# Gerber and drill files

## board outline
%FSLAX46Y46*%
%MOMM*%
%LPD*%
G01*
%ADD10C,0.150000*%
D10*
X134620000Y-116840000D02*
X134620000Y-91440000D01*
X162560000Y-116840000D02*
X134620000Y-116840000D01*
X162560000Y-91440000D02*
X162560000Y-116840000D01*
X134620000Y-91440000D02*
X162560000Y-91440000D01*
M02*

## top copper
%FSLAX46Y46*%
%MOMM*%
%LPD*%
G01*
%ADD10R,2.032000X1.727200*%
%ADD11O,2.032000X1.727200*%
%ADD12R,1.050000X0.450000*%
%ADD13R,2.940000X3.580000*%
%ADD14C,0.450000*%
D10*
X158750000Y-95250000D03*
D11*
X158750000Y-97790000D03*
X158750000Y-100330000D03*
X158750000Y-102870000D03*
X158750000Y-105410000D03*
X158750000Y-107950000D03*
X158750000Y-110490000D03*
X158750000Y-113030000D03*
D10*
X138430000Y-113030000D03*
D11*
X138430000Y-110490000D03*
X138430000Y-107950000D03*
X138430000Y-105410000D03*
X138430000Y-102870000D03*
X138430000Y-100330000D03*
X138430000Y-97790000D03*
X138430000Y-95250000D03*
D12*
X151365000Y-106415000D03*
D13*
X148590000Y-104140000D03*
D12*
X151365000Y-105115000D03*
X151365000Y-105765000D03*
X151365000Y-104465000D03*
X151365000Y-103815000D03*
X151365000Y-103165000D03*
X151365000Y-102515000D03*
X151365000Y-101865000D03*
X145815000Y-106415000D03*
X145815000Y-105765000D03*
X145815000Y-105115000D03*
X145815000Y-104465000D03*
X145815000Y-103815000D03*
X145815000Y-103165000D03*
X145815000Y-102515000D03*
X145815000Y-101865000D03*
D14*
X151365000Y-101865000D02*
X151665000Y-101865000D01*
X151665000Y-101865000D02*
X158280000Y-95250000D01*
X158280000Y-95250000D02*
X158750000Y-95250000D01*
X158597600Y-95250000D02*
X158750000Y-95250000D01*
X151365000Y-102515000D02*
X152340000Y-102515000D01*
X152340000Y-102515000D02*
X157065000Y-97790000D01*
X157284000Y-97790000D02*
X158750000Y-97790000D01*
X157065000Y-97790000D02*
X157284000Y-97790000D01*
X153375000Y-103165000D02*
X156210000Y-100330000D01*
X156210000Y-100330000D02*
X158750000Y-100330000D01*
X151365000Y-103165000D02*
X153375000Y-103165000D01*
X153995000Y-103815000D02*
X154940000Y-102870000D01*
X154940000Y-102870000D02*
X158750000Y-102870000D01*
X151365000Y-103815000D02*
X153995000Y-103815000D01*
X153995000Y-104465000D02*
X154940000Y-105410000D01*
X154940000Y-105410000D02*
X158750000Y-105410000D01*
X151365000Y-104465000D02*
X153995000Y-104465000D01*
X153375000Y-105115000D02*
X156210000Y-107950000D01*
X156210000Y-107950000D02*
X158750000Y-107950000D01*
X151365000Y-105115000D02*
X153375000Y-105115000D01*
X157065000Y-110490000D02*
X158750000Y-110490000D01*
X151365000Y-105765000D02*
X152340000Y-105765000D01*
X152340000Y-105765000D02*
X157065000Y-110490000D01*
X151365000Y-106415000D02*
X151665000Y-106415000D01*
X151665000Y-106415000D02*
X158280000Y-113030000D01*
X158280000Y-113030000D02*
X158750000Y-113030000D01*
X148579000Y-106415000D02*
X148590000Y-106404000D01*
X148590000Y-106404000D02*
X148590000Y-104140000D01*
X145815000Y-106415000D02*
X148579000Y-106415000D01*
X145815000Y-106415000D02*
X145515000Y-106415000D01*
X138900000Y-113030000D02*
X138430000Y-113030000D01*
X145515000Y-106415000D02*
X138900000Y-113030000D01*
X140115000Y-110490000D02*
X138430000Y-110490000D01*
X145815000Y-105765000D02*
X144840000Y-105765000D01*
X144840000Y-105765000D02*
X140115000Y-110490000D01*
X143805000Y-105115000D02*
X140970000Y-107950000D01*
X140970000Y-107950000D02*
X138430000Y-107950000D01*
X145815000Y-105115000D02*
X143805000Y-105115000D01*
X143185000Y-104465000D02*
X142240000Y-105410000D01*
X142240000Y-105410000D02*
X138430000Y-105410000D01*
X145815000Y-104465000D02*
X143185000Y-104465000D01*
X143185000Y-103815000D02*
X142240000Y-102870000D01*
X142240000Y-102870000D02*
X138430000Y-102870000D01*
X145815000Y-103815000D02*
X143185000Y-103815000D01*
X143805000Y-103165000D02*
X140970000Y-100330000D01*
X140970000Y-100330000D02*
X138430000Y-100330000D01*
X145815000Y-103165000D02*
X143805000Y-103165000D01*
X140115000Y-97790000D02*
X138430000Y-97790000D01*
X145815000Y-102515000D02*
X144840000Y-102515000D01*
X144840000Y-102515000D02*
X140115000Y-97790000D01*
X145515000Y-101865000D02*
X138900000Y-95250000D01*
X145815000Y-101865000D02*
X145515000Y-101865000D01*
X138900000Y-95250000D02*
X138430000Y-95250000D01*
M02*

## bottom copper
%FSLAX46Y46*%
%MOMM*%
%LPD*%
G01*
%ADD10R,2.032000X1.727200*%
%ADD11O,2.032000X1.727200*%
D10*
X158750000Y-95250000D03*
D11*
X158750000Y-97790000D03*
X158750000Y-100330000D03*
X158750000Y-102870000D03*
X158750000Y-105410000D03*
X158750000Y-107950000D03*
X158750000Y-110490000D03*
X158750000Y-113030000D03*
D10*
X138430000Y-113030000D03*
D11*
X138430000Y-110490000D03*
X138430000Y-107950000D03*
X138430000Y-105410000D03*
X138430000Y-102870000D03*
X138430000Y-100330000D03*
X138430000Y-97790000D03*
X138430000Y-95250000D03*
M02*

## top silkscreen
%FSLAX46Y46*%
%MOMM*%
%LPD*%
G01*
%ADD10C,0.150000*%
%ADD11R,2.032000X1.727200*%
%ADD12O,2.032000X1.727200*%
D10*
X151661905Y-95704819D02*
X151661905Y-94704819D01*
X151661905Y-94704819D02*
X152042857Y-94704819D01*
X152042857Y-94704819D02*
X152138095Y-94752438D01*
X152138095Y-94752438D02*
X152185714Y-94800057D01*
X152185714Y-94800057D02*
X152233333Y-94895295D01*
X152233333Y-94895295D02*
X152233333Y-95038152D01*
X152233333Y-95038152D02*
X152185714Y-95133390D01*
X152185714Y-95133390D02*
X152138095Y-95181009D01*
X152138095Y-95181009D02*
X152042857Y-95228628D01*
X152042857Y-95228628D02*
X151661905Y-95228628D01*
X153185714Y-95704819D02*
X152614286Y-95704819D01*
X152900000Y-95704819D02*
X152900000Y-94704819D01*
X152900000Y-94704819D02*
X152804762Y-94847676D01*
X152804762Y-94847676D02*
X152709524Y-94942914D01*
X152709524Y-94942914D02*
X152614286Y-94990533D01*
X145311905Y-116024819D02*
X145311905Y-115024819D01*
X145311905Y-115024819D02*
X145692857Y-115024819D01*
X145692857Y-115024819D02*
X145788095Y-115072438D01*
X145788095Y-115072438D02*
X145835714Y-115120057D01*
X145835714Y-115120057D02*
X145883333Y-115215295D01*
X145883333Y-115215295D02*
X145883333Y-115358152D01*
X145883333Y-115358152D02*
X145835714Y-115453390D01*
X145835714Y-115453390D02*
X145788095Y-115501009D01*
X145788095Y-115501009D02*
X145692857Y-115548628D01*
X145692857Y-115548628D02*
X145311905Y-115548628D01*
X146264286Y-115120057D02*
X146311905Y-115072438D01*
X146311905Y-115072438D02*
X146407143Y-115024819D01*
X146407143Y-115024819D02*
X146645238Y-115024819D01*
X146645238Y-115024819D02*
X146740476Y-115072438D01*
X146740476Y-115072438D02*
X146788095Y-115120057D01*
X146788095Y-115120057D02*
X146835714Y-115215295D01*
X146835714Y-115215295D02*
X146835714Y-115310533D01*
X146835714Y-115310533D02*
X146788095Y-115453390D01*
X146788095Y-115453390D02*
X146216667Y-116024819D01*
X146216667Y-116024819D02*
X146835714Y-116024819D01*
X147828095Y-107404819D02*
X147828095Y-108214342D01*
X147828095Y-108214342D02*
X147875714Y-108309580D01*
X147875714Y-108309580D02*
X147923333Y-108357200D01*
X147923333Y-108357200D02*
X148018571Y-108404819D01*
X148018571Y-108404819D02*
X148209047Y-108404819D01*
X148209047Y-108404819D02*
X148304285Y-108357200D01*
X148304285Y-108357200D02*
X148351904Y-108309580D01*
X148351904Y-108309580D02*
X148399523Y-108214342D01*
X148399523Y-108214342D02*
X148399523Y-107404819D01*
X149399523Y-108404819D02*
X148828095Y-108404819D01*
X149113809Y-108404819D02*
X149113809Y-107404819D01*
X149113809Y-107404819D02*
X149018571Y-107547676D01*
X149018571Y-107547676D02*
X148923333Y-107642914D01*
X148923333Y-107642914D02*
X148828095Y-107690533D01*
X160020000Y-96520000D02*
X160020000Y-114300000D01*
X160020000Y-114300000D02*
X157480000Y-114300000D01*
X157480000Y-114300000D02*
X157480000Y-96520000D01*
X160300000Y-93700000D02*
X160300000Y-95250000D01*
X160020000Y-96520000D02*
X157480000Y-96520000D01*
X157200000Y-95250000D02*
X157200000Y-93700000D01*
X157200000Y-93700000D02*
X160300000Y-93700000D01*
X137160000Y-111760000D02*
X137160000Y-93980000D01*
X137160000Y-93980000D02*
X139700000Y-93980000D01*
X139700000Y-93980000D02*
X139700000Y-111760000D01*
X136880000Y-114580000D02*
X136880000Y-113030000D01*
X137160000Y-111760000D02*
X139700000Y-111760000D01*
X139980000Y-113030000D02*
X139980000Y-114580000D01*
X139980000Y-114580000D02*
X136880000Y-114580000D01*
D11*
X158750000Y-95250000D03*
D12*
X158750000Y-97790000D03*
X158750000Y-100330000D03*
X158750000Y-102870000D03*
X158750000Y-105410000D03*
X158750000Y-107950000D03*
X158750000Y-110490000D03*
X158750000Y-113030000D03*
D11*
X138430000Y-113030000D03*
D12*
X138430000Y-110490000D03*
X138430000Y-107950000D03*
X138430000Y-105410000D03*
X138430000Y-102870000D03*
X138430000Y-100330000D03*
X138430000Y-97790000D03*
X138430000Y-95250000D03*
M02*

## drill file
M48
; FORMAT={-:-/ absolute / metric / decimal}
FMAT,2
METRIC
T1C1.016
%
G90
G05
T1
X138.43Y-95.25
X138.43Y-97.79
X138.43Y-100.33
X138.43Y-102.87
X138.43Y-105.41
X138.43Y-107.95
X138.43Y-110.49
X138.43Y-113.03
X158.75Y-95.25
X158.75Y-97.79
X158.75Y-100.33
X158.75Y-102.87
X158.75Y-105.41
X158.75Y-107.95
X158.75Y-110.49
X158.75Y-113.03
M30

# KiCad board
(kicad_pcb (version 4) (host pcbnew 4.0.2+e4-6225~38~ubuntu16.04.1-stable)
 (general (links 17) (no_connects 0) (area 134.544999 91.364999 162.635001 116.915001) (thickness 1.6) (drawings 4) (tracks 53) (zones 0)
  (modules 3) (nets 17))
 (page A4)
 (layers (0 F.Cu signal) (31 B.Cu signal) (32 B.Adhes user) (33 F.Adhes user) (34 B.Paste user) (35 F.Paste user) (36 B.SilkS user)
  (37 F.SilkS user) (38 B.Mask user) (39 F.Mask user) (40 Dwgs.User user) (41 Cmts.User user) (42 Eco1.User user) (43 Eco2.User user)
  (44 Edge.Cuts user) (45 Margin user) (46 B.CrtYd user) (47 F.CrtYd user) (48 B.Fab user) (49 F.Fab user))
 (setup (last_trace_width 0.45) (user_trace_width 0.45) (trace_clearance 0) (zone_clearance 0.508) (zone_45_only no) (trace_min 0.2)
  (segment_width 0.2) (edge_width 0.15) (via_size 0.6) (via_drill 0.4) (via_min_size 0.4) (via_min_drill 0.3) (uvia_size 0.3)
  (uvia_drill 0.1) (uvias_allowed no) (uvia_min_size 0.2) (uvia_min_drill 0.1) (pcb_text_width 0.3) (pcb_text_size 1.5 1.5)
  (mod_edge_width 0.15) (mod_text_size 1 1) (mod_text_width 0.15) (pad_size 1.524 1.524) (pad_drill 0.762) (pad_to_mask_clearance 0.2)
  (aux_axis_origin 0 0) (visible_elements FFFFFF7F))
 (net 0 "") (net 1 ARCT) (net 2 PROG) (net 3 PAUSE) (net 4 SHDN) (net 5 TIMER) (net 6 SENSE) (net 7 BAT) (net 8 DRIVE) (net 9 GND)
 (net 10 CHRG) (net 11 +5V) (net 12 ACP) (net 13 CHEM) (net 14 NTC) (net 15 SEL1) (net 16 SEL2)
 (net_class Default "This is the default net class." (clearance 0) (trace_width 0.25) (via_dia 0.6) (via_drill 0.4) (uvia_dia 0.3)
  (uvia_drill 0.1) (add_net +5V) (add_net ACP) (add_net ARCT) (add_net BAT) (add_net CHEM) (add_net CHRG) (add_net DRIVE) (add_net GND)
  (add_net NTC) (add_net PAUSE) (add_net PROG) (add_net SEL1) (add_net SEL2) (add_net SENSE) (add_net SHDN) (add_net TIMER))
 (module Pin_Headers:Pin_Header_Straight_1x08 (layer F.Cu) (at 158.75 95.25)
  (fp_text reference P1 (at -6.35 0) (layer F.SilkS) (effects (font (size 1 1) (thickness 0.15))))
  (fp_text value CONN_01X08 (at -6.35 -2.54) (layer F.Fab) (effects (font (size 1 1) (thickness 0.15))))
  (fp_line (start 1.27 1.27) (end 1.27 19.05) (layer F.SilkS) (width 0.15))
  (fp_line (start 1.27 19.05) (end -1.27 19.05) (layer F.SilkS) (width 0.15))
  (fp_line (start -1.27 19.05) (end -1.27 1.27) (layer F.SilkS) (width 0.15))
  (fp_line (start 1.55 -1.55) (end 1.55 0) (layer F.SilkS) (width 0.15))
  (fp_line (start 1.27 1.27) (end -1.27 1.27) (layer F.SilkS) (width 0.15))
  (fp_line (start -1.55 0) (end -1.55 -1.55) (layer F.SilkS) (width 0.15))
  (fp_line (start -1.55 -1.55) (end 1.55 -1.55) (layer F.SilkS) (width 0.15))
  (pad 1 thru_hole rect (at 0 0) (size 2.032 1.7272) (drill 1.016) (layers *.Cu *.Mask F.SilkS) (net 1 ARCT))
  (pad 2 thru_hole oval (at 0 2.54) (size 2.032 1.7272) (drill 1.016) (layers *.Cu *.Mask F.SilkS) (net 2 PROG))
  (pad 3 thru_hole oval (at 0 5.08) (size 2.032 1.7272) (drill 1.016) (layers *.Cu *.Mask F.SilkS) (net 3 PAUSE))
  (pad 4 thru_hole oval (at 0 7.62) (size 2.032 1.7272) (drill 1.016) (layers *.Cu *.Mask F.SilkS) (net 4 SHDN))
  (pad 5 thru_hole oval (at 0 10.16) (size 2.032 1.7272) (drill 1.016) (layers *.Cu *.Mask F.SilkS) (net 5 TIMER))
  (pad 6 thru_hole oval (at 0 12.7) (size 2.032 1.7272) (drill 1.016) (layers *.Cu *.Mask F.SilkS) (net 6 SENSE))
  (pad 7 thru_hole oval (at 0 15.24) (size 2.032 1.7272) (drill 1.016) (layers *.Cu *.Mask F.SilkS) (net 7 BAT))
  (pad 8 thru_hole oval (at 0 17.78) (size 2.032 1.7272) (drill 1.016) (layers *.Cu *.Mask F.SilkS) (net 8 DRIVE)))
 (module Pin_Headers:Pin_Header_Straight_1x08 (layer F.Cu) (at 138.43 113.03 180)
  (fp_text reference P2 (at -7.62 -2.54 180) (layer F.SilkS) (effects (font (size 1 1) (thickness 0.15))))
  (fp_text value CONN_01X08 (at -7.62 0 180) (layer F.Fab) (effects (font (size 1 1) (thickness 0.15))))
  (fp_line (start 1.27 1.27) (end 1.27 19.05) (layer F.SilkS) (width 0.15))
  (fp_line (start 1.27 19.05) (end -1.27 19.05) (layer F.SilkS) (width 0.15))
  (fp_line (start -1.27 19.05) (end -1.27 1.27) (layer F.SilkS) (width 0.15))
  (fp_line (start 1.55 -1.55) (end 1.55 0) (layer F.SilkS) (width 0.15))
  (fp_line (start 1.27 1.27) (end -1.27 1.27) (layer F.SilkS) (width 0.15))
  (fp_line (start -1.55 0) (end -1.55 -1.55) (layer F.SilkS) (width 0.15))
  (fp_line (start -1.55 -1.55) (end 1.55 -1.55) (layer F.SilkS) (width 0.15))
  (pad 1 thru_hole rect (at 0 0 180) (size 2.032 1.7272) (drill 1.016) (layers *.Cu *.Mask F.SilkS) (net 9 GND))
  (pad 2 thru_hole oval (at 0 2.54 180) (size 2.032 1.7272) (drill 1.016) (layers *.Cu *.Mask F.SilkS) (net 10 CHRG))
  (pad 3 thru_hole oval (at 0 5.08 180) (size 2.032 1.7272) (drill 1.016) (layers *.Cu *.Mask F.SilkS) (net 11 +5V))
  (pad 4 thru_hole oval (at 0 7.62 180) (size 2.032 1.7272) (drill 1.016) (layers *.Cu *.Mask F.SilkS) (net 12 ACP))
  (pad 5 thru_hole oval (at 0 10.16 180) (size 2.032 1.7272) (drill 1.016) (layers *.Cu *.Mask F.SilkS) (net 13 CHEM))
  (pad 6 thru_hole oval (at 0 12.7 180) (size 2.032 1.7272) (drill 1.016) (layers *.Cu *.Mask F.SilkS) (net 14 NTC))
  (pad 7 thru_hole oval (at 0 15.24 180) (size 2.032 1.7272) (drill 1.016) (layers *.Cu *.Mask F.SilkS) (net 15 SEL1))
  (pad 8 thru_hole oval (at 0 17.78 180) (size 2.032 1.7272) (drill 1.016) (layers *.Cu *.Mask F.SilkS) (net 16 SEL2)))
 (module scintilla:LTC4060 (layer F.Cu) (at 148.59 104.14 90)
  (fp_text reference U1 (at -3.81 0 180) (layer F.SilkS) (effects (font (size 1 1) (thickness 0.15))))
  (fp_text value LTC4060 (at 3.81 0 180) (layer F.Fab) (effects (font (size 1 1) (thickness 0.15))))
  (pad 1 smd rect (at -2.275 2.775 90) (size 0.45 1.05) (layers F.Cu F.Paste F.Mask) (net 8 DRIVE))
  (pad 17 smd rect (at 0 0 90) (size 3.58 2.94) (layers F.Cu F.Paste F.Mask) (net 9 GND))
  (pad 3 smd rect (at -0.975 2.775 90) (size 0.45 1.05) (layers F.Cu F.Paste F.Mask) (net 6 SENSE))
  (pad 2 smd rect (at -1.625 2.775 90) (size 0.45 1.05) (layers F.Cu F.Paste F.Mask) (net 7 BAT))
  (pad 4 smd rect (at -0.325 2.775 90) (size 0.45 1.05) (layers F.Cu F.Paste F.Mask) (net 5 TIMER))
  (pad 5 smd rect (at 0.325 2.775 90) (size 0.45 1.05) (layers F.Cu F.Paste F.Mask) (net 4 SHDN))
  (pad 6 smd rect (at 0.975 2.775 90) (size 0.45 1.05) (layers F.Cu F.Paste F.Mask) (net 3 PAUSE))
  (pad 7 smd rect (at 1.625 2.775 90) (size 0.45 1.05) (layers F.Cu F.Paste F.Mask) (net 2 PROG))
  (pad 8 smd rect (at 2.275 2.775 90) (size 0.45 1.05) (layers F.Cu F.Paste F.Mask) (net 1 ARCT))
  (pad 16 smd rect (at -2.275 -2.775 90) (size 0.45 1.05) (layers F.Cu F.Paste F.Mask) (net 9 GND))
  (pad 15 smd rect (at -1.625 -2.775 90) (size 0.45 1.05) (layers F.Cu F.Paste F.Mask) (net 10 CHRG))
  (pad 14 smd rect (at -0.975 -2.775 90) (size 0.45 1.05) (layers F.Cu F.Paste F.Mask) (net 11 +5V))
  (pad 13 smd rect (at -0.325 -2.775 90) (size 0.45 1.05) (layers F.Cu F.Paste F.Mask) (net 12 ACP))
  (pad 12 smd rect (at 0.325 -2.775 90) (size 0.45 1.05) (layers F.Cu F.Paste F.Mask) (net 13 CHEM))
  (pad 11 smd rect (at 0.975 -2.775 90) (size 0.45 1.05) (layers F.Cu F.Paste F.Mask) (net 14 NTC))
  (pad 10 smd rect (at 1.625 -2.775 90) (size 0.45 1.05) (layers F.Cu F.Paste F.Mask) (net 15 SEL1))
  (pad 9 smd rect (at 2.275 -2.775 90) (size 0.45 1.05) (layers F.Cu F.Paste F.Mask) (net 16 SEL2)))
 (gr_line (start 134.62 116.84) (end 134.62 91.44) (layer Edge.Cuts) (width 0.15))
 (gr_line (start 162.56 116.84) (end 134.62 116.84) (layer Edge.Cuts) (width 0.15))
 (gr_line (start 162.56 91.44) (end 162.56 116.84) (layer Edge.Cuts) (width 0.15))
 (gr_line (start 134.62 91.44) (end 162.56 91.44) (layer Edge.Cuts) (width 0.15))
 (segment (start 151.365 101.865) (end 151.665 101.865) (width 0.45) (layer F.Cu) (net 1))
 (segment (start 151.665 101.865) (end 158.28 95.25) (width 0.45) (layer F.Cu) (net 1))
 (segment (start 158.28 95.25) (end 158.75 95.25) (width 0.45) (layer F.Cu) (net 1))
 (segment (start 158.5976 95.25) (end 158.75 95.25) (width 0.45) (layer F.Cu) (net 1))
 (segment (start 151.365 102.515) (end 152.34 102.515) (width 0.45) (layer F.Cu) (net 2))
 (segment (start 152.34 102.515) (end 157.065 97.79) (width 0.45) (layer F.Cu) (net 2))
 (segment (start 157.284 97.79) (end 158.75 97.79) (width 0.45) (layer F.Cu) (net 2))
 (segment (start 157.065 97.79) (end 157.284 97.79) (width 0.45) (layer F.Cu) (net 2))
 (segment (start 153.375 103.165) (end 156.21 100.33) (width 0.45) (layer F.Cu) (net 3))
 (segment (start 156.21 100.33) (end 158.75 100.33) (width 0.45) (layer F.Cu) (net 3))
 (segment (start 151.365 103.165) (end 153.375 103.165) (width 0.45) (layer F.Cu) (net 3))
 (segment (start 153.995 103.815) (end 154.94 102.87) (width 0.45) (layer F.Cu) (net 4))
 (segment (start 154.94 102.87) (end 158.75 102.87) (width 0.45) (layer F.Cu) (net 4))
 (segment (start 151.365 103.815) (end 153.995 103.815) (width 0.45) (layer F.Cu) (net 4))
 (segment (start 153.995 104.465) (end 154.94 105.41) (width 0.45) (layer F.Cu) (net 5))
 (segment (start 154.94 105.41) (end 158.75 105.41) (width 0.45) (layer F.Cu) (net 5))
 (segment (start 151.365 104.465) (end 153.995 104.465) (width 0.45) (layer F.Cu) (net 5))
 (segment (start 153.375 105.115) (end 156.21 107.95) (width 0.45) (layer F.Cu) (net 6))
 (segment (start 156.21 107.95) (end 158.75 107.95) (width 0.45) (layer F.Cu) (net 6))
 (segment (start 151.365 105.115) (end 153.375 105.115) (width 0.45) (layer F.Cu) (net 6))
 (segment (start 157.065 110.49) (end 158.75 110.49) (width 0.45) (layer F.Cu) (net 7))
 (segment (start 151.365 105.765) (end 152.34 105.765) (width 0.45) (layer F.Cu) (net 7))
 (segment (start 152.34 105.765) (end 157.065 110.49) (width 0.45) (layer F.Cu) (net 7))
 (segment (start 151.365 106.415) (end 151.665 106.415) (width 0.45) (layer F.Cu) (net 8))
 (segment (start 151.665 106.415) (end 158.28 113.03) (width 0.45) (layer F.Cu) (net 8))
 (segment (start 158.28 113.03) (end 158.75 113.03) (width 0.45) (layer F.Cu) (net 8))
 (segment (start 148.579 106.415) (end 148.59 106.404) (width 0.45) (layer F.Cu) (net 9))
 (segment (start 148.59 106.404) (end 148.59 104.14) (width 0.45) (layer F.Cu) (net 9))
 (segment (start 145.815 106.415) (end 148.579 106.415) (width 0.45) (layer F.Cu) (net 9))
 (segment (start 145.815 106.415) (end 145.515 106.415) (width 0.45) (layer F.Cu) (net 9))
 (segment (start 138.9 113.03) (end 138.43 113.03) (width 0.45) (layer F.Cu) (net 9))
 (segment (start 145.515 106.415) (end 138.9 113.03) (width 0.45) (layer F.Cu) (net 9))
 (segment (start 140.115 110.49) (end 138.43 110.49) (width 0.45) (layer F.Cu) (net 10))
 (segment (start 145.815 105.765) (end 144.84 105.765) (width 0.45) (layer F.Cu) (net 10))
 (segment (start 144.84 105.765) (end 140.115 110.49) (width 0.45) (layer F.Cu) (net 10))
 (segment (start 143.805 105.115) (end 140.97 107.95) (width 0.45) (layer F.Cu) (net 11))
 (segment (start 140.97 107.95) (end 138.43 107.95) (width 0.45) (layer F.Cu) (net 11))
 (segment (start 145.815 105.115) (end 143.805 105.115) (width 0.45) (layer F.Cu) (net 11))
 (segment (start 143.185 104.465) (end 142.24 105.41) (width 0.45) (layer F.Cu) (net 12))
 (segment (start 142.24 105.41) (end 138.43 105.41) (width 0.45) (layer F.Cu) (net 12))
 (segment (start 145.815 104.465) (end 143.185 104.465) (width 0.45) (layer F.Cu) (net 12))
 (segment (start 143.185 103.815) (end 142.24 102.87) (width 0.45) (layer F.Cu) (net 13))
 (segment (start 142.24 102.87) (end 138.43 102.87) (width 0.45) (layer F.Cu) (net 13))
 (segment (start 145.815 103.815) (end 143.185 103.815) (width 0.45) (layer F.Cu) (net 13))
 (segment (start 143.805 103.165) (end 140.97 100.33) (width 0.45) (layer F.Cu) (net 14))
 (segment (start 140.97 100.33) (end 138.43 100.33) (width 0.45) (layer F.Cu) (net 14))
 (segment (start 145.815 103.165) (end 143.805 103.165) (width 0.45) (layer F.Cu) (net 14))
 (segment (start 140.115 97.79) (end 138.43 97.79) (width 0.45) (layer F.Cu) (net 15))
 (segment (start 145.815 102.515) (end 144.84 102.515) (width 0.45) (layer F.Cu) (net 15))
 (segment (start 144.84 102.515) (end 140.115 97.79) (width 0.45) (layer F.Cu) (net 15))
 (segment (start 145.515 101.865) (end 138.9 95.25) (width 0.45) (layer F.Cu) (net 16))
 (segment (start 145.815 101.865) (end 145.515 101.865) (width 0.45) (layer F.Cu) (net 16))
 (segment (start 138.9 95.25) (end 138.43 95.25) (width 0.45) (layer F.Cu) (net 16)))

